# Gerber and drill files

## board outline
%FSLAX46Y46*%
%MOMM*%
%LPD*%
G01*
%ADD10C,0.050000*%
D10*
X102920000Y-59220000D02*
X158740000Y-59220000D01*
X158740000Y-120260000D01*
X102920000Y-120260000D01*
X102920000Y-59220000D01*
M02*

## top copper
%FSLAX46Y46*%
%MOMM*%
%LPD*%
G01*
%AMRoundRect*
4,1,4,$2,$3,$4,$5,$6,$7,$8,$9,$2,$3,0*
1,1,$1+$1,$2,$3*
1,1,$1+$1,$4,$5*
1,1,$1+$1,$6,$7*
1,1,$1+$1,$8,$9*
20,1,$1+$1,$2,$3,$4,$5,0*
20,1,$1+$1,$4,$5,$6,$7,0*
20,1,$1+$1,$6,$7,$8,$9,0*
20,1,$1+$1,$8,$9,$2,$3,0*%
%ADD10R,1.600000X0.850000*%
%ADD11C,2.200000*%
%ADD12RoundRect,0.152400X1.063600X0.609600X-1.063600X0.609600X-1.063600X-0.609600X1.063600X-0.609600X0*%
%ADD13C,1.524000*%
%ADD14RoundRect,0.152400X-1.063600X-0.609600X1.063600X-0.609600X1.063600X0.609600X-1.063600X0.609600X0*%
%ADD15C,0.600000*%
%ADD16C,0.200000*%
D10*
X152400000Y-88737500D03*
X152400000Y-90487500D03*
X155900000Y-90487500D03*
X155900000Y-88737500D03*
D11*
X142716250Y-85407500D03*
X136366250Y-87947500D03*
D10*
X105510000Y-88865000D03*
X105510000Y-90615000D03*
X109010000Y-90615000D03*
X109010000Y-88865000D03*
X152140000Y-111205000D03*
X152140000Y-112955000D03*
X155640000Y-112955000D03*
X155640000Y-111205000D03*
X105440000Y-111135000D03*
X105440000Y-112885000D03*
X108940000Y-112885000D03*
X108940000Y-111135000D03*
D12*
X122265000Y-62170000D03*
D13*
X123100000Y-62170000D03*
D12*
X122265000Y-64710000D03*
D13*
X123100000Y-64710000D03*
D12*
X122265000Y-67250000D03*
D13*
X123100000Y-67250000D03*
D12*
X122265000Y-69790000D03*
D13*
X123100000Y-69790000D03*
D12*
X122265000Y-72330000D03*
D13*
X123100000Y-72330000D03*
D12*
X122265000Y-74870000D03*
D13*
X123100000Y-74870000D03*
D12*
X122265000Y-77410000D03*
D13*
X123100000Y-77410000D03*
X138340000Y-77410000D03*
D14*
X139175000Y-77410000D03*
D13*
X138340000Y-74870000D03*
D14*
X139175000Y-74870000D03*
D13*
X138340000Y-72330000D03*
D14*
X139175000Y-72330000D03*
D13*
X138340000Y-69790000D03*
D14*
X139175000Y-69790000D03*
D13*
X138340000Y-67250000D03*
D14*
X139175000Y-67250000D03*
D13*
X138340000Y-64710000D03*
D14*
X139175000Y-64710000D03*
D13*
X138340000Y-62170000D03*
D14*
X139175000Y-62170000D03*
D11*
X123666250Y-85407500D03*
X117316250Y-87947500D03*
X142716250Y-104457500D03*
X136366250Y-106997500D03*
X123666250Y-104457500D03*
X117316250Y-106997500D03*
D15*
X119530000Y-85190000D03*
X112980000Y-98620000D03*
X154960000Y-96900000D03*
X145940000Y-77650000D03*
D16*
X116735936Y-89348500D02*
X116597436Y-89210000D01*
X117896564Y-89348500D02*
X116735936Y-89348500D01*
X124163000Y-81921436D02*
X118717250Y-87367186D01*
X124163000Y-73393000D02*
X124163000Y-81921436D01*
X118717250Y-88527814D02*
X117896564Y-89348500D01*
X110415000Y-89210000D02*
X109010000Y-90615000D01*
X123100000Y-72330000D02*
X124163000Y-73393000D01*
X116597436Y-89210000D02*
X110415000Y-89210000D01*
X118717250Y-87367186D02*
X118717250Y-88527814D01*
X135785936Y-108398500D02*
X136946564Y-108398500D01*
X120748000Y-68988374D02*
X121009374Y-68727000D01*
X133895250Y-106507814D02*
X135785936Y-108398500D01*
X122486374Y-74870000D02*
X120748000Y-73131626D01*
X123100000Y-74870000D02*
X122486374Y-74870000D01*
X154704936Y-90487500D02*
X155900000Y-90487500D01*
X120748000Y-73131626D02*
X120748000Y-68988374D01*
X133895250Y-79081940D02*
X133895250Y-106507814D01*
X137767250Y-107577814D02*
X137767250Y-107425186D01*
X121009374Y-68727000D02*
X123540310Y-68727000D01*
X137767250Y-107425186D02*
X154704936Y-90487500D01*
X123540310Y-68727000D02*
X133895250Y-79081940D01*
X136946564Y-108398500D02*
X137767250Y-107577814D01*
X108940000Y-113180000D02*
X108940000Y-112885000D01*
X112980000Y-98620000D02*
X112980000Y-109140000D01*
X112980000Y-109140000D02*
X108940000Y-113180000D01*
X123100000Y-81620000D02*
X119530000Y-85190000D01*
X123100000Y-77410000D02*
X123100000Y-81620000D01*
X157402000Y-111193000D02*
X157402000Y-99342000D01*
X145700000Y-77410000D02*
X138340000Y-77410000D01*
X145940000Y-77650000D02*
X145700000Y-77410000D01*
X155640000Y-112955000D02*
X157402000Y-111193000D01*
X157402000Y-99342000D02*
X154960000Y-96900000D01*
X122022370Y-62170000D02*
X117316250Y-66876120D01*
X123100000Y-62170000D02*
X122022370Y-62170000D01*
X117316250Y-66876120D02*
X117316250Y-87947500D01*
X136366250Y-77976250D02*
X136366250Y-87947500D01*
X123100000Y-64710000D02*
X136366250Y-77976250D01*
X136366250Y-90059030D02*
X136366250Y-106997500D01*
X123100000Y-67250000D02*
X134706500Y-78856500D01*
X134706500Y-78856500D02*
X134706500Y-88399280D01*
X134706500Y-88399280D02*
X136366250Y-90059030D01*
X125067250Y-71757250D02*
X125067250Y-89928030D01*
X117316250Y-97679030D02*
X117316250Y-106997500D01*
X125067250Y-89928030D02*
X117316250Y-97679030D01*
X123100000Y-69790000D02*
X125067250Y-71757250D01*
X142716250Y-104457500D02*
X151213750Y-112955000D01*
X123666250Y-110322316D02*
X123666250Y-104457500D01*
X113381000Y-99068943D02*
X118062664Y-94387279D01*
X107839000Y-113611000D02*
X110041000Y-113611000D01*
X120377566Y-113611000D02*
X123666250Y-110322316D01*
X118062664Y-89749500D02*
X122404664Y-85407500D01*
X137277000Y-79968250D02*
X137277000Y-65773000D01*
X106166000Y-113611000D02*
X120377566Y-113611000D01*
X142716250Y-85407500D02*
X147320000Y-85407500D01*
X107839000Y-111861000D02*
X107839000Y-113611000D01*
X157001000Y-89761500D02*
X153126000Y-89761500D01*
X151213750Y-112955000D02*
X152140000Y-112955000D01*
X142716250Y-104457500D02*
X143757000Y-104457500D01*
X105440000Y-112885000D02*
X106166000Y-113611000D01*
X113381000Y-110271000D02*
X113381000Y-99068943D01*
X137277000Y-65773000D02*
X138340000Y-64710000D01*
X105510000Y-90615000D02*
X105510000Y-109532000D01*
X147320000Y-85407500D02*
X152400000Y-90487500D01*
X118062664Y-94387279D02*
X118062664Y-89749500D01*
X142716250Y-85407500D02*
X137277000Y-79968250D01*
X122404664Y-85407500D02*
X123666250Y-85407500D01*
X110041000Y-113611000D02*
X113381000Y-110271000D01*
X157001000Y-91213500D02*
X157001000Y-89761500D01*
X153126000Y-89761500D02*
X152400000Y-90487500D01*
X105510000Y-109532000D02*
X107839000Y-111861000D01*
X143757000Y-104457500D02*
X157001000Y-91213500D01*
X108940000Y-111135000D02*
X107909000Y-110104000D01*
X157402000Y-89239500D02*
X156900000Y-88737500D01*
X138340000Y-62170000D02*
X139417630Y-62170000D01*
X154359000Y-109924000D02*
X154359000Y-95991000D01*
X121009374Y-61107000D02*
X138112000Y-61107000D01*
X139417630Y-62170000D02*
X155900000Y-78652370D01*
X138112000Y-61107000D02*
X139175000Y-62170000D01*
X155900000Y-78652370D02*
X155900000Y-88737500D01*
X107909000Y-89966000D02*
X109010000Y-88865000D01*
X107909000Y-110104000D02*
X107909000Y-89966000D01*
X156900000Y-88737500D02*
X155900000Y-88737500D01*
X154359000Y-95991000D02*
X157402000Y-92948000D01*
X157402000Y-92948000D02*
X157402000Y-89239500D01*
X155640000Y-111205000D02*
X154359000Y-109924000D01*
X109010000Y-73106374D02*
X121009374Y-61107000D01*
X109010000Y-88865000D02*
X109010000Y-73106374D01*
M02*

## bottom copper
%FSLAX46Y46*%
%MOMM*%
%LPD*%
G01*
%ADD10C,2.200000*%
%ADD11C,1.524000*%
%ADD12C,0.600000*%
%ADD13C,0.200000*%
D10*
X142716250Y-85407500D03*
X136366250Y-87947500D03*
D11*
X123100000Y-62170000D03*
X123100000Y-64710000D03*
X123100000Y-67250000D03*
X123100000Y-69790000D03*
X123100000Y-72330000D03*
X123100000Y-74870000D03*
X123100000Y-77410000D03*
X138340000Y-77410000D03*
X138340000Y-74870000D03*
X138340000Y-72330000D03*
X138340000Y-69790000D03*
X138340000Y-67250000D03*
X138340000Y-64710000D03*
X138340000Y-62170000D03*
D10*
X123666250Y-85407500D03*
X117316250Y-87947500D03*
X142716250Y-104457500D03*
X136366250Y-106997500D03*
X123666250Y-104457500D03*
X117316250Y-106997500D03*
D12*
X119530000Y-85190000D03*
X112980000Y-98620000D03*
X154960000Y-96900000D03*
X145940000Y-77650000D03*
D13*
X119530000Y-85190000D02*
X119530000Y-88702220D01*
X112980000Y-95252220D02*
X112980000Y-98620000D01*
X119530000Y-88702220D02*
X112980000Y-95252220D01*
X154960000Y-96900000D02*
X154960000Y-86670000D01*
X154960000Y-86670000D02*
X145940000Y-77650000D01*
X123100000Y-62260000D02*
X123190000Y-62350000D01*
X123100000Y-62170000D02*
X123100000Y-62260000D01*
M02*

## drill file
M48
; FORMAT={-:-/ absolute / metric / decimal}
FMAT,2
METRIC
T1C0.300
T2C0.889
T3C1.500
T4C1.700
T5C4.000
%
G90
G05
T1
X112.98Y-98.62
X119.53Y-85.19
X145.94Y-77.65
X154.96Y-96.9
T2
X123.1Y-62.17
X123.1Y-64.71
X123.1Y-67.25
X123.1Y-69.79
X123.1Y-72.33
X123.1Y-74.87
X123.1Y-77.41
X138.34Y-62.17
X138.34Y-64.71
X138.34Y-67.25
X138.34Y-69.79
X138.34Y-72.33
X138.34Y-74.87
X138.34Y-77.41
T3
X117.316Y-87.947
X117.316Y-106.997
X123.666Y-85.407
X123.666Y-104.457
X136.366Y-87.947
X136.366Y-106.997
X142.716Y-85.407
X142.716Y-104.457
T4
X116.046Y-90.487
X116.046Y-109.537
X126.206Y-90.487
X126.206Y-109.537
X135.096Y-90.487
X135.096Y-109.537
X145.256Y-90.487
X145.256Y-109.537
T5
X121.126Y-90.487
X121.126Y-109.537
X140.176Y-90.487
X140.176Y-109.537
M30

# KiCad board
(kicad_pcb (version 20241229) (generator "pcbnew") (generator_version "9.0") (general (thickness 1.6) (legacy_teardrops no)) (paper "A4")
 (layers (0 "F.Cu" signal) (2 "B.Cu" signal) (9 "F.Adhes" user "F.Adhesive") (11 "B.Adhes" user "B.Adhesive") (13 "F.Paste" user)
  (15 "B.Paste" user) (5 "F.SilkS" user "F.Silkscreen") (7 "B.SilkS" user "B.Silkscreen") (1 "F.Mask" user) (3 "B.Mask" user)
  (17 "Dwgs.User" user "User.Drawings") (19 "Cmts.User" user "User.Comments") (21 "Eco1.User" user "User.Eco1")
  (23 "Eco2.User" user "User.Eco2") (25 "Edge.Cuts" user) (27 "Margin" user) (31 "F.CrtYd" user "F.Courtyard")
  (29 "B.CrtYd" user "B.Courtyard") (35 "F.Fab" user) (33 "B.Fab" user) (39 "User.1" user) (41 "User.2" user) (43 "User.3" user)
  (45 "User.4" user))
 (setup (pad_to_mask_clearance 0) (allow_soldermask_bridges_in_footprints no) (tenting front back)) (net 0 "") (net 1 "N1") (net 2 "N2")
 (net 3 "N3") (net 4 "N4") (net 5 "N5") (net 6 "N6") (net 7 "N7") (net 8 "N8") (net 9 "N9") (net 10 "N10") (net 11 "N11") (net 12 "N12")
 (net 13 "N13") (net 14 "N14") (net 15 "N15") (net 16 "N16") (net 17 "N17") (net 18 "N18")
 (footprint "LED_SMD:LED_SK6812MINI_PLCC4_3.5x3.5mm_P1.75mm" (layer "F.Cu") (at 154.15 89.6125)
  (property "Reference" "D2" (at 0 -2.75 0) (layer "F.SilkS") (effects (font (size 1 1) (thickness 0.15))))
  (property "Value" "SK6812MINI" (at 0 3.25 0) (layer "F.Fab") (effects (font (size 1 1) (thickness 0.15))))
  (pad "1" smd rect (at -1.75 -0.875) (size 1.6 0.85) (layers "F.Cu" "F.Mask" "F.Paste") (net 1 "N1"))
  (pad "2" smd rect (at -1.75 0.875) (size 1.6 0.85) (layers "F.Cu" "F.Mask" "F.Paste") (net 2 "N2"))
  (pad "3" smd rect (at 1.75 0.875) (size 1.6 0.85) (layers "F.Cu" "F.Mask" "F.Paste") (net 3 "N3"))
  (pad "4" smd rect (at 1.75 -0.875) (size 1.6 0.85) (layers "F.Cu" "F.Mask" "F.Paste") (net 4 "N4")))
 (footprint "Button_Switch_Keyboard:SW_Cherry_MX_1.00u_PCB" (layer "F.Cu") (at 142.71625 85.4075)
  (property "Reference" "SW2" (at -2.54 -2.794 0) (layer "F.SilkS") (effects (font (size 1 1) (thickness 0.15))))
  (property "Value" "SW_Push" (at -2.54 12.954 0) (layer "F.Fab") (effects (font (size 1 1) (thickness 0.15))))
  (pad "" np_thru_hole circle (at -7.62 5.08) (size 1.7 1.7) (drill 1.7) (layers "*.Cu" "*.Mask"))
  (pad "" np_thru_hole circle (at -2.54 5.08) (size 4 4) (drill 4) (layers "*.Cu" "*.Mask"))
  (pad "" np_thru_hole circle (at 2.54 5.08) (size 1.7 1.7) (drill 1.7) (layers "*.Cu" "*.Mask"))
  (pad "1" thru_hole circle (at 0 0) (size 2.2 2.2) (drill 1.5) (layers "*.Cu" "*.Mask") (remove_unused_layers no) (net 2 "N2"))
  (pad "2" thru_hole circle (at -6.35 2.54) (size 2.2 2.2) (drill 1.5) (layers "*.Cu" "*.Mask") (remove_unused_layers no) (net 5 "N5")))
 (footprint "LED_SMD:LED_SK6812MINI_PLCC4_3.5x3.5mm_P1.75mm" (layer "F.Cu") (at 107.26 89.74)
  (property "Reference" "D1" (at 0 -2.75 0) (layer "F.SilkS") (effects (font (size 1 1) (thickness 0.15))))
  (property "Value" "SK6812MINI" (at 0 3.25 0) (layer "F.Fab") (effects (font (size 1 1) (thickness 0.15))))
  (pad "1" smd rect (at -1.75 -0.875) (size 1.6 0.85) (layers "F.Cu" "F.Mask" "F.Paste") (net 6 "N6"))
  (pad "2" smd rect (at -1.75 0.875) (size 1.6 0.85) (layers "F.Cu" "F.Mask" "F.Paste") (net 2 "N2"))
  (pad "3" smd rect (at 1.75 0.875) (size 1.6 0.85) (layers "F.Cu" "F.Mask" "F.Paste") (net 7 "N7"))
  (pad "4" smd rect (at 1.75 -0.875) (size 1.6 0.85) (layers "F.Cu" "F.Mask" "F.Paste") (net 4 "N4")))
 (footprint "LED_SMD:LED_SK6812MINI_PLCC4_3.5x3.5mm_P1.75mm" (layer "F.Cu") (at 153.89 112.08)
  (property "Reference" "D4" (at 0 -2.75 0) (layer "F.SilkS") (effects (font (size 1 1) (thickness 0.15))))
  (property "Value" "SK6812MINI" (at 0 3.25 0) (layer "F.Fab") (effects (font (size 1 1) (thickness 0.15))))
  (pad "1" smd rect (at -1.75 -0.875) (size 1.6 0.85) (layers "F.Cu" "F.Mask" "F.Paste") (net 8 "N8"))
  (pad "2" smd rect (at -1.75 0.875) (size 1.6 0.85) (layers "F.Cu" "F.Mask" "F.Paste") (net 2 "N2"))
  (pad "3" smd rect (at 1.75 0.875) (size 1.6 0.85) (layers "F.Cu" "F.Mask" "F.Paste") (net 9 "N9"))
  (pad "4" smd rect (at 1.75 -0.875) (size 1.6 0.85) (layers "F.Cu" "F.Mask" "F.Paste") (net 4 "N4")))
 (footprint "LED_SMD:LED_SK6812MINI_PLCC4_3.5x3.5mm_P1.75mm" (layer "F.Cu") (at 107.19 112.01)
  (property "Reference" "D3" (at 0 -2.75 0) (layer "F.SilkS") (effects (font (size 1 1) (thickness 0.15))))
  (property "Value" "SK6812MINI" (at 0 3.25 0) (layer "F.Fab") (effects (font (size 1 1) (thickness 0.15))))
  (pad "1" smd rect (at -1.75 -0.875) (size 1.6 0.85) (layers "F.Cu" "F.Mask" "F.Paste") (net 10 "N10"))
  (pad "2" smd rect (at -1.75 0.875) (size 1.6 0.85) (layers "F.Cu" "F.Mask" "F.Paste") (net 2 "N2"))
  (pad "3" smd rect (at 1.75 0.875) (size 1.6 0.85) (layers "F.Cu" "F.Mask" "F.Paste") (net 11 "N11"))
  (pad "4" smd rect (at 1.75 -0.875) (size 1.6 0.85) (layers "F.Cu" "F.Mask" "F.Paste") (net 4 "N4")))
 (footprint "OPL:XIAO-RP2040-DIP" (layer "F.Cu") (at 130.72 69.79)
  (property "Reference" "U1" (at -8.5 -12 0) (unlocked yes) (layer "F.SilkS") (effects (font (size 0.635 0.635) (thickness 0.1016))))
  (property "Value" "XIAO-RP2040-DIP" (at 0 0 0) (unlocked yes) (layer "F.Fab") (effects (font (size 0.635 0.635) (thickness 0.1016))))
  (pad "1" smd roundrect (at -8.455 -7.62 180) (size 2.432 1.524) (layers "F.Cu" "F.Mask") (roundrect_rratio 0.1) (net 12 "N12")
   (thermal_bridge_angle 45))
  (pad "1" thru_hole circle (at -7.62 -7.62 180) (size 1.524 1.524) (drill 0.889) (layers "*.Cu" "*.Mask") (remove_unused_layers no)
   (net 12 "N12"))
  (pad "2" smd roundrect (at -8.455 -5.08 180) (size 2.432 1.524) (layers "F.Cu" "F.Mask") (roundrect_rratio 0.1) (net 5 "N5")
   (thermal_bridge_angle 45))
  (pad "2" thru_hole circle (at -7.62 -5.08 180) (size 1.524 1.524) (drill 0.889) (layers "*.Cu" "*.Mask") (remove_unused_layers no)
   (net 5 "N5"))
  (pad "3" smd roundrect (at -8.455 -2.54 180) (size 2.432 1.524) (layers "F.Cu" "F.Mask") (roundrect_rratio 0.1) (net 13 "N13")
   (thermal_bridge_angle 45))
  (pad "3" thru_hole circle (at -7.62 -2.54 180) (size 1.524 1.524) (drill 0.889) (layers "*.Cu" "*.Mask") (remove_unused_layers no)
   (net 13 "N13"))
  (pad "4" smd roundrect (at -8.455 0 180) (size 2.432 1.524) (layers "F.Cu" "F.Mask") (roundrect_rratio 0.1) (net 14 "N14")
   (thermal_bridge_angle 45))
  (pad "4" thru_hole circle (at -7.62 0 180) (size 1.524 1.524) (drill 0.889) (layers "*.Cu" "*.Mask") (remove_unused_layers no)
   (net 14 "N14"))
  (pad "5" smd roundrect (at -8.455 2.54 180) (size 2.432 1.524) (layers "F.Cu" "F.Mask") (roundrect_rratio 0.1) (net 7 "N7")
   (thermal_bridge_angle 45))
  (pad "5" thru_hole circle (at -7.62 2.54 180) (size 1.524 1.524) (drill 0.889) (layers "*.Cu" "*.Mask") (remove_unused_layers no)
   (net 7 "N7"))
  (pad "6" smd roundrect (at -8.455 5.08 180) (size 2.432 1.524) (layers "F.Cu" "F.Mask") (roundrect_rratio 0.1) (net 3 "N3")
   (thermal_bridge_angle 45))
  (pad "6" thru_hole circle (at -7.62 5.08 180) (size 1.524 1.524) (drill 0.889) (layers "*.Cu" "*.Mask") (remove_unused_layers no)
   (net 3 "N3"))
  (pad "7" smd roundrect (at -8.455 7.62 180) (size 2.432 1.524) (layers "F.Cu" "F.Mask") (roundrect_rratio 0.1) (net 11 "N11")
   (thermal_bridge_angle 45))
  (pad "7" thru_hole circle (at -7.62 7.62 180) (size 1.524 1.524) (drill 0.889) (layers "*.Cu" "*.Mask") (remove_unused_layers no)
   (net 11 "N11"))
  (pad "8" thru_hole circle (at 7.62 7.62) (size 1.524 1.524) (drill 0.889) (layers "*.Cu" "*.Mask") (remove_unused_layers no) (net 9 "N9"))
  (pad "8" smd roundrect (at 8.455 7.62) (size 2.432 1.524) (layers "F.Cu" "F.Mask") (roundrect_rratio 0.1) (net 9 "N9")
   (thermal_bridge_angle 45))
  (pad "9" thru_hole circle (at 7.62 5.08) (size 1.524 1.524) (drill 0.889) (layers "*.Cu" "*.Mask") (remove_unused_layers no)
   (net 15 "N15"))
  (pad "9" smd roundrect (at 8.455 5.08) (size 2.432 1.524) (layers "F.Cu" "F.Mask") (roundrect_rratio 0.1) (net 15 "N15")
   (thermal_bridge_angle 45))
  (pad "10" thru_hole circle (at 7.62 2.54) (size 1.524 1.524) (drill 0.889) (layers "*.Cu" "*.Mask") (remove_unused_layers no)
   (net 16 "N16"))
  (pad "10" smd roundrect (at 8.455 2.54) (size 2.432 1.524) (layers "F.Cu" "F.Mask") (roundrect_rratio 0.1) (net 16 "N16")
   (thermal_bridge_angle 45))
  (pad "11" thru_hole circle (at 7.62 0) (size 1.524 1.524) (drill 0.889) (layers "*.Cu" "*.Mask") (remove_unused_layers no) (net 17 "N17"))
  (pad "11" smd roundrect (at 8.455 0) (size 2.432 1.524) (layers "F.Cu" "F.Mask") (roundrect_rratio 0.1) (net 17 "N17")
   (thermal_bridge_angle 45))
  (pad "12" thru_hole circle (at 7.62 -2.54) (size 1.524 1.524) (drill 0.889) (layers "*.Cu" "*.Mask") (remove_unused_layers no)
   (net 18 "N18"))
  (pad "12" smd roundrect (at 8.455 -2.54) (size 2.432 1.524) (layers "F.Cu" "F.Mask") (roundrect_rratio 0.1) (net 18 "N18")
   (thermal_bridge_angle 45))
  (pad "13" thru_hole circle (at 7.62 -5.08) (size 1.524 1.524) (drill 0.889) (layers "*.Cu" "*.Mask") (remove_unused_layers no)
   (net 2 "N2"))
  (pad "13" smd roundrect (at 8.455 -5.08) (size 2.432 1.524) (layers "F.Cu" "F.Mask") (roundrect_rratio 0.1) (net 2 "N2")
   (thermal_bridge_angle 45))
  (pad "14" thru_hole circle (at 7.62 -7.62) (size 1.524 1.524) (drill 0.889) (layers "*.Cu" "*.Mask") (remove_unused_layers no)
   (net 4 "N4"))
  (pad "14" smd roundrect (at 8.455 -7.62) (size 2.432 1.524) (layers "F.Cu" "F.Mask") (roundrect_rratio 0.1) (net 4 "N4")
   (thermal_bridge_angle 45)))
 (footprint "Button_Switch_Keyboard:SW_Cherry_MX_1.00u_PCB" (layer "F.Cu") (at 123.66625 85.4075)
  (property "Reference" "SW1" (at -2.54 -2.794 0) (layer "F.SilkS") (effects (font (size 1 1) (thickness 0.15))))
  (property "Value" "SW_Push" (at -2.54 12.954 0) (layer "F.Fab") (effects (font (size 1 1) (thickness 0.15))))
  (pad "" np_thru_hole circle (at -7.62 5.08) (size 1.7 1.7) (drill 1.7) (layers "*.Cu" "*.Mask"))
  (pad "" np_thru_hole circle (at -2.54 5.08) (size 4 4) (drill 4) (layers "*.Cu" "*.Mask"))
  (pad "" np_thru_hole circle (at 2.54 5.08) (size 1.7 1.7) (drill 1.7) (layers "*.Cu" "*.Mask"))
  (pad "1" thru_hole circle (at 0 0) (size 2.2 2.2) (drill 1.5) (layers "*.Cu" "*.Mask") (remove_unused_layers no) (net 2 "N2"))
  (pad "2" thru_hole circle (at -6.35 2.54) (size 2.2 2.2) (drill 1.5) (layers "*.Cu" "*.Mask") (remove_unused_layers no) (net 12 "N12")))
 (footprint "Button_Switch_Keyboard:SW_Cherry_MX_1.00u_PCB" (layer "F.Cu") (at 142.71625 104.4575)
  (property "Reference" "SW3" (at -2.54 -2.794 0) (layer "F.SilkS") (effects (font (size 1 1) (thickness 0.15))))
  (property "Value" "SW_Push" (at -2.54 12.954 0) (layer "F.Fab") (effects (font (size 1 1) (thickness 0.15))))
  (pad "" np_thru_hole circle (at -7.62 5.08) (size 1.7 1.7) (drill 1.7) (layers "*.Cu" "*.Mask"))
  (pad "" np_thru_hole circle (at -2.54 5.08) (size 4 4) (drill 4) (layers "*.Cu" "*.Mask"))
  (pad "" np_thru_hole circle (at 2.54 5.08) (size 1.7 1.7) (drill 1.7) (layers "*.Cu" "*.Mask"))
  (pad "1" thru_hole circle (at 0 0) (size 2.2 2.2) (drill 1.5) (layers "*.Cu" "*.Mask") (remove_unused_layers no) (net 2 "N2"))
  (pad "2" thru_hole circle (at -6.35 2.54) (size 2.2 2.2) (drill 1.5) (layers "*.Cu" "*.Mask") (remove_unused_layers no) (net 13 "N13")))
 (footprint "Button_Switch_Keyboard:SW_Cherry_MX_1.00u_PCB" (layer "F.Cu") (at 123.66625 104.4575)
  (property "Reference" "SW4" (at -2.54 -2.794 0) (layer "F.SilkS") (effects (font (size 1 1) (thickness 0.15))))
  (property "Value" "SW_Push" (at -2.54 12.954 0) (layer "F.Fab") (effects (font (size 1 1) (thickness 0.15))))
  (pad "" np_thru_hole circle (at -7.62 5.08) (size 1.7 1.7) (drill 1.7) (layers "*.Cu" "*.Mask"))
  (pad "" np_thru_hole circle (at -2.54 5.08) (size 4 4) (drill 4) (layers "*.Cu" "*.Mask"))
  (pad "" np_thru_hole circle (at 2.54 5.08) (size 1.7 1.7) (drill 1.7) (layers "*.Cu" "*.Mask"))
  (pad "1" thru_hole circle (at 0 0) (size 2.2 2.2) (drill 1.5) (layers "*.Cu" "*.Mask") (remove_unused_layers no) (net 2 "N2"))
  (pad "2" thru_hole circle (at -6.35 2.54) (size 2.2 2.2) (drill 1.5) (layers "*.Cu" "*.Mask") (remove_unused_layers no) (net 14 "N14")))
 (gr_rect (start 102.92 59.22) (end 158.74 120.26) (stroke (width 0.05) (type default)) (fill no) (layer "Edge.Cuts"))
 (segment (start 116.735936 89.3485) (end 116.597436 89.21) (width 0.2) (layer "F.Cu") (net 7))
 (segment (start 117.896564 89.3485) (end 116.735936 89.3485) (width 0.2) (layer "F.Cu") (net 7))
 (segment (start 124.163 81.921436) (end 118.71725 87.367186) (width 0.2) (layer "F.Cu") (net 7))
 (segment (start 124.163 73.393) (end 124.163 81.921436) (width 0.2) (layer "F.Cu") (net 7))
 (segment (start 118.71725 88.527814) (end 117.896564 89.3485) (width 0.2) (layer "F.Cu") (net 7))
 (segment (start 110.415 89.21) (end 109.01 90.615) (width 0.2) (layer "F.Cu") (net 7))
 (segment (start 123.1 72.33) (end 124.163 73.393) (width 0.2) (layer "F.Cu") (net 7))
 (segment (start 116.597436 89.21) (end 110.415 89.21) (width 0.2) (layer "F.Cu") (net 7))
 (segment (start 118.71725 87.367186) (end 118.71725 88.527814) (width 0.2) (layer "F.Cu") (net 7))
 (segment (start 135.785936 108.3985) (end 136.946564 108.3985) (width 0.2) (layer "F.Cu") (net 3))
 (segment (start 120.748 68.988374) (end 121.009374 68.727) (width 0.2) (layer "F.Cu") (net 3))
 (segment (start 133.89525 106.507814) (end 135.785936 108.3985) (width 0.2) (layer "F.Cu") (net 3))
 (segment (start 122.486374 74.87) (end 120.748 73.131626) (width 0.2) (layer "F.Cu") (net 3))
 (segment (start 123.1 74.87) (end 122.486374 74.87) (width 0.2) (layer "F.Cu") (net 3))
 (segment (start 154.704936 90.4875) (end 155.9 90.4875) (width 0.2) (layer "F.Cu") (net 3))
 (segment (start 120.748 73.131626) (end 120.748 68.988374) (width 0.2) (layer "F.Cu") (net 3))
 (segment (start 133.89525 79.08194) (end 133.89525 106.507814) (width 0.2) (layer "F.Cu") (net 3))
 (segment (start 137.76725 107.577814) (end 137.76725 107.425186) (width 0.2) (layer "F.Cu") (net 3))
 (segment (start 121.009374 68.727) (end 123.54031 68.727) (width 0.2) (layer "F.Cu") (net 3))
 (segment (start 137.76725 107.425186) (end 154.704936 90.4875) (width 0.2) (layer "F.Cu") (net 3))
 (segment (start 123.54031 68.727) (end 133.89525 79.08194) (width 0.2) (layer "F.Cu") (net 3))
 (segment (start 136.946564 108.3985) (end 137.76725 107.577814) (width 0.2) (layer "F.Cu") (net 3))
 (segment (start 108.94 113.18) (end 108.94 112.885) (width 0.2) (layer "F.Cu") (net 11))
 (segment (start 112.98 98.62) (end 112.98 109.14) (width 0.2) (layer "F.Cu") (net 11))
 (segment (start 112.98 109.14) (end 108.94 113.18) (width 0.2) (layer "F.Cu") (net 11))
 (segment (start 123.1 81.62) (end 119.53 85.19) (width 0.2) (layer "F.Cu") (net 11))
 (segment (start 123.1 77.41) (end 123.1 81.62) (width 0.2) (layer "F.Cu") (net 11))
 (via (at 119.53 85.19) (size 0.6) (drill 0.3) (layers "F.Cu" "B.Cu") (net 11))
 (via (at 112.98 98.62) (size 0.6) (drill 0.3) (layers "F.Cu" "B.Cu") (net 11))
 (segment (start 119.53 85.19) (end 119.53 88.70222) (width 0.2) (layer "B.Cu") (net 11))
 (segment (start 112.98 95.25222) (end 112.98 98.62) (width 0.2) (layer "B.Cu") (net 11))
 (segment (start 119.53 88.70222) (end 112.98 95.25222) (width 0.2) (layer "B.Cu") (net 11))
 (segment (start 157.402 111.193) (end 157.402 99.342) (width 0.2) (layer "F.Cu") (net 9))
 (segment (start 145.7 77.41) (end 138.34 77.41) (width 0.2) (layer "F.Cu") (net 9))
 (segment (start 145.94 77.65) (end 145.7 77.41) (width 0.2) (layer "F.Cu") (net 9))
 (segment (start 155.64 112.955) (end 157.402 111.193) (width 0.2) (layer "F.Cu") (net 9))
 (segment (start 157.402 99.342) (end 154.96 96.9) (width 0.2) (layer "F.Cu") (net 9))
 (via (at 154.96 96.9) (size 0.6) (drill 0.3) (layers "F.Cu" "B.Cu") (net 9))
 (via (at 145.94 77.65) (size 0.6) (drill 0.3) (layers "F.Cu" "B.Cu") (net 9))
 (segment (start 154.96 96.9) (end 154.96 86.67) (width 0.2) (layer "B.Cu") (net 9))
 (segment (start 154.96 86.67) (end 145.94 77.65) (width 0.2) (layer "B.Cu") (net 9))
 (segment (start 122.02237 62.17) (end 117.31625 66.87612) (width 0.2) (layer "F.Cu") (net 12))
 (segment (start 123.1 62.17) (end 122.02237 62.17) (width 0.2) (layer "F.Cu") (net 12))
 (segment (start 117.31625 66.87612) (end 117.31625 87.9475) (width 0.2) (layer "F.Cu") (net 12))
 (segment (start 123.1 62.26) (end 123.19 62.35) (width 0.2) (layer "B.Cu") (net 12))
 (segment (start 123.1 62.17) (end 123.1 62.26) (width 0.2) (layer "B.Cu") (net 12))
 (segment (start 136.36625 77.97625) (end 136.36625 87.9475) (width 0.2) (layer "F.Cu") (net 5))
 (segment (start 123.1 64.71) (end 136.36625 77.97625) (width 0.2) (layer "F.Cu") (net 5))
 (segment (start 136.36625 90.05903) (end 136.36625 106.9975) (width 0.2) (layer "F.Cu") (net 13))
 (segment (start 123.1 67.25) (end 134.7065 78.8565) (width 0.2) (layer "F.Cu") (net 13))
 (segment (start 134.7065 78.8565) (end 134.7065 88.39928) (width 0.2) (layer "F.Cu") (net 13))
 (segment (start 134.7065 88.39928) (end 136.36625 90.05903) (width 0.2) (layer "F.Cu") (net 13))
 (segment (start 125.06725 71.75725) (end 125.06725 89.92803) (width 0.2) (layer "F.Cu") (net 14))
 (segment (start 117.31625 97.67903) (end 117.31625 106.9975) (width 0.2) (layer "F.Cu") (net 14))
 (segment (start 125.06725 89.92803) (end 117.31625 97.67903) (width 0.2) (layer "F.Cu") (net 14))
 (segment (start 123.1 69.79) (end 125.06725 71.75725) (width 0.2) (layer "F.Cu") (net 14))
 (segment (start 142.71625 104.4575) (end 151.21375 112.955) (width 0.2) (layer "F.Cu") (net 2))
 (segment (start 123.66625 110.322316) (end 123.66625 104.4575) (width 0.2) (layer "F.Cu") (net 2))
 (segment (start 113.381 99.068943) (end 118.062664 94.387279) (width 0.2) (layer "F.Cu") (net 2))
 (segment (start 107.839 113.611) (end 110.041 113.611) (width 0.2) (layer "F.Cu") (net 2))
 (segment (start 120.377566 113.611) (end 123.66625 110.322316) (width 0.2) (layer "F.Cu") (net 2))
 (segment (start 118.062664 89.7495) (end 122.404664 85.4075) (width 0.2) (layer "F.Cu") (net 2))
 (segment (start 137.277 79.96825) (end 137.277 65.773) (width 0.2) (layer "F.Cu") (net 2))
 (segment (start 106.166 113.611) (end 120.377566 113.611) (width 0.2) (layer "F.Cu") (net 2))
 (segment (start 142.71625 85.4075) (end 147.32 85.4075) (width 0.2) (layer "F.Cu") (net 2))
 (segment (start 107.839 111.861) (end 107.839 113.611) (width 0.2) (layer "F.Cu") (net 2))
 (segment (start 157.001 89.7615) (end 153.126 89.7615) (width 0.2) (layer "F.Cu") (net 2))
 (segment (start 151.21375 112.955) (end 152.14 112.955) (width 0.2) (layer "F.Cu") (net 2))
 (segment (start 142.71625 104.4575) (end 143.757 104.4575) (width 0.2) (layer "F.Cu") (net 2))
 (segment (start 105.44 112.885) (end 106.166 113.611) (width 0.2) (layer "F.Cu") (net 2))
 (segment (start 113.381 110.271) (end 113.381 99.068943) (width 0.2) (layer "F.Cu") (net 2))
 (segment (start 137.277 65.773) (end 138.34 64.71) (width 0.2) (layer "F.Cu") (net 2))
 (segment (start 105.51 90.615) (end 105.51 109.532) (width 0.2) (layer "F.Cu") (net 2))
 (segment (start 147.32 85.4075) (end 152.4 90.4875) (width 0.2) (layer "F.Cu") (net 2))
 (segment (start 118.062664 94.387279) (end 118.062664 89.7495) (width 0.2) (layer "F.Cu") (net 2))
 (segment (start 142.71625 85.4075) (end 137.277 79.96825) (width 0.2) (layer "F.Cu") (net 2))
 (segment (start 122.404664 85.4075) (end 123.66625 85.4075) (width 0.2) (layer "F.Cu") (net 2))
 (segment (start 110.041 113.611) (end 113.381 110.271) (width 0.2) (layer "F.Cu") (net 2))
 (segment (start 157.001 91.2135) (end 157.001 89.7615) (width 0.2) (layer "F.Cu") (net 2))
 (segment (start 153.126 89.7615) (end 152.4 90.4875) (width 0.2) (layer "F.Cu") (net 2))
 (segment (start 105.51 109.532) (end 107.839 111.861) (width 0.2) (layer "F.Cu") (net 2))
 (segment (start 143.757 104.4575) (end 157.001 91.2135) (width 0.2) (layer "F.Cu") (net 2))
 (segment (start 108.94 111.135) (end 107.909 110.104) (width 0.2) (layer "F.Cu") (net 4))
 (segment (start 157.402 89.2395) (end 156.9 88.7375) (width 0.2) (layer "F.Cu") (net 4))
 (segment (start 138.34 62.17) (end 139.41763 62.17) (width 0.2) (layer "F.Cu") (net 4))
 (segment (start 154.359 109.924) (end 154.359 95.991) (width 0.2) (layer "F.Cu") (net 4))
 (segment (start 121.009374 61.107) (end 138.112 61.107) (width 0.2) (layer "F.Cu") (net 4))
 (segment (start 139.41763 62.17) (end 155.9 78.65237) (width 0.2) (layer "F.Cu") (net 4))
 (segment (start 138.112 61.107) (end 139.175 62.17) (width 0.2) (layer "F.Cu") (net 4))
 (segment (start 155.9 78.65237) (end 155.9 88.7375) (width 0.2) (layer "F.Cu") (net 4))
 (segment (start 107.909 89.966) (end 109.01 88.865) (width 0.2) (layer "F.Cu") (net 4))
 (segment (start 107.909 110.104) (end 107.909 89.966) (width 0.2) (layer "F.Cu") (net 4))
 (segment (start 156.9 88.7375) (end 155.9 88.7375) (width 0.2) (layer "F.Cu") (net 4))
 (segment (start 154.359 95.991) (end 157.402 92.948) (width 0.2) (layer "F.Cu") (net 4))
 (segment (start 157.402 92.948) (end 157.402 89.2395) (width 0.2) (layer "F.Cu") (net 4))
 (segment (start 155.64 111.205) (end 154.359 109.924) (width 0.2) (layer "F.Cu") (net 4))
 (segment (start 109.01 73.106374) (end 121.009374 61.107) (width 0.2) (layer "F.Cu") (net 4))
 (segment (start 109.01 88.865) (end 109.01 73.106374) (width 0.2) (layer "F.Cu") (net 4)))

